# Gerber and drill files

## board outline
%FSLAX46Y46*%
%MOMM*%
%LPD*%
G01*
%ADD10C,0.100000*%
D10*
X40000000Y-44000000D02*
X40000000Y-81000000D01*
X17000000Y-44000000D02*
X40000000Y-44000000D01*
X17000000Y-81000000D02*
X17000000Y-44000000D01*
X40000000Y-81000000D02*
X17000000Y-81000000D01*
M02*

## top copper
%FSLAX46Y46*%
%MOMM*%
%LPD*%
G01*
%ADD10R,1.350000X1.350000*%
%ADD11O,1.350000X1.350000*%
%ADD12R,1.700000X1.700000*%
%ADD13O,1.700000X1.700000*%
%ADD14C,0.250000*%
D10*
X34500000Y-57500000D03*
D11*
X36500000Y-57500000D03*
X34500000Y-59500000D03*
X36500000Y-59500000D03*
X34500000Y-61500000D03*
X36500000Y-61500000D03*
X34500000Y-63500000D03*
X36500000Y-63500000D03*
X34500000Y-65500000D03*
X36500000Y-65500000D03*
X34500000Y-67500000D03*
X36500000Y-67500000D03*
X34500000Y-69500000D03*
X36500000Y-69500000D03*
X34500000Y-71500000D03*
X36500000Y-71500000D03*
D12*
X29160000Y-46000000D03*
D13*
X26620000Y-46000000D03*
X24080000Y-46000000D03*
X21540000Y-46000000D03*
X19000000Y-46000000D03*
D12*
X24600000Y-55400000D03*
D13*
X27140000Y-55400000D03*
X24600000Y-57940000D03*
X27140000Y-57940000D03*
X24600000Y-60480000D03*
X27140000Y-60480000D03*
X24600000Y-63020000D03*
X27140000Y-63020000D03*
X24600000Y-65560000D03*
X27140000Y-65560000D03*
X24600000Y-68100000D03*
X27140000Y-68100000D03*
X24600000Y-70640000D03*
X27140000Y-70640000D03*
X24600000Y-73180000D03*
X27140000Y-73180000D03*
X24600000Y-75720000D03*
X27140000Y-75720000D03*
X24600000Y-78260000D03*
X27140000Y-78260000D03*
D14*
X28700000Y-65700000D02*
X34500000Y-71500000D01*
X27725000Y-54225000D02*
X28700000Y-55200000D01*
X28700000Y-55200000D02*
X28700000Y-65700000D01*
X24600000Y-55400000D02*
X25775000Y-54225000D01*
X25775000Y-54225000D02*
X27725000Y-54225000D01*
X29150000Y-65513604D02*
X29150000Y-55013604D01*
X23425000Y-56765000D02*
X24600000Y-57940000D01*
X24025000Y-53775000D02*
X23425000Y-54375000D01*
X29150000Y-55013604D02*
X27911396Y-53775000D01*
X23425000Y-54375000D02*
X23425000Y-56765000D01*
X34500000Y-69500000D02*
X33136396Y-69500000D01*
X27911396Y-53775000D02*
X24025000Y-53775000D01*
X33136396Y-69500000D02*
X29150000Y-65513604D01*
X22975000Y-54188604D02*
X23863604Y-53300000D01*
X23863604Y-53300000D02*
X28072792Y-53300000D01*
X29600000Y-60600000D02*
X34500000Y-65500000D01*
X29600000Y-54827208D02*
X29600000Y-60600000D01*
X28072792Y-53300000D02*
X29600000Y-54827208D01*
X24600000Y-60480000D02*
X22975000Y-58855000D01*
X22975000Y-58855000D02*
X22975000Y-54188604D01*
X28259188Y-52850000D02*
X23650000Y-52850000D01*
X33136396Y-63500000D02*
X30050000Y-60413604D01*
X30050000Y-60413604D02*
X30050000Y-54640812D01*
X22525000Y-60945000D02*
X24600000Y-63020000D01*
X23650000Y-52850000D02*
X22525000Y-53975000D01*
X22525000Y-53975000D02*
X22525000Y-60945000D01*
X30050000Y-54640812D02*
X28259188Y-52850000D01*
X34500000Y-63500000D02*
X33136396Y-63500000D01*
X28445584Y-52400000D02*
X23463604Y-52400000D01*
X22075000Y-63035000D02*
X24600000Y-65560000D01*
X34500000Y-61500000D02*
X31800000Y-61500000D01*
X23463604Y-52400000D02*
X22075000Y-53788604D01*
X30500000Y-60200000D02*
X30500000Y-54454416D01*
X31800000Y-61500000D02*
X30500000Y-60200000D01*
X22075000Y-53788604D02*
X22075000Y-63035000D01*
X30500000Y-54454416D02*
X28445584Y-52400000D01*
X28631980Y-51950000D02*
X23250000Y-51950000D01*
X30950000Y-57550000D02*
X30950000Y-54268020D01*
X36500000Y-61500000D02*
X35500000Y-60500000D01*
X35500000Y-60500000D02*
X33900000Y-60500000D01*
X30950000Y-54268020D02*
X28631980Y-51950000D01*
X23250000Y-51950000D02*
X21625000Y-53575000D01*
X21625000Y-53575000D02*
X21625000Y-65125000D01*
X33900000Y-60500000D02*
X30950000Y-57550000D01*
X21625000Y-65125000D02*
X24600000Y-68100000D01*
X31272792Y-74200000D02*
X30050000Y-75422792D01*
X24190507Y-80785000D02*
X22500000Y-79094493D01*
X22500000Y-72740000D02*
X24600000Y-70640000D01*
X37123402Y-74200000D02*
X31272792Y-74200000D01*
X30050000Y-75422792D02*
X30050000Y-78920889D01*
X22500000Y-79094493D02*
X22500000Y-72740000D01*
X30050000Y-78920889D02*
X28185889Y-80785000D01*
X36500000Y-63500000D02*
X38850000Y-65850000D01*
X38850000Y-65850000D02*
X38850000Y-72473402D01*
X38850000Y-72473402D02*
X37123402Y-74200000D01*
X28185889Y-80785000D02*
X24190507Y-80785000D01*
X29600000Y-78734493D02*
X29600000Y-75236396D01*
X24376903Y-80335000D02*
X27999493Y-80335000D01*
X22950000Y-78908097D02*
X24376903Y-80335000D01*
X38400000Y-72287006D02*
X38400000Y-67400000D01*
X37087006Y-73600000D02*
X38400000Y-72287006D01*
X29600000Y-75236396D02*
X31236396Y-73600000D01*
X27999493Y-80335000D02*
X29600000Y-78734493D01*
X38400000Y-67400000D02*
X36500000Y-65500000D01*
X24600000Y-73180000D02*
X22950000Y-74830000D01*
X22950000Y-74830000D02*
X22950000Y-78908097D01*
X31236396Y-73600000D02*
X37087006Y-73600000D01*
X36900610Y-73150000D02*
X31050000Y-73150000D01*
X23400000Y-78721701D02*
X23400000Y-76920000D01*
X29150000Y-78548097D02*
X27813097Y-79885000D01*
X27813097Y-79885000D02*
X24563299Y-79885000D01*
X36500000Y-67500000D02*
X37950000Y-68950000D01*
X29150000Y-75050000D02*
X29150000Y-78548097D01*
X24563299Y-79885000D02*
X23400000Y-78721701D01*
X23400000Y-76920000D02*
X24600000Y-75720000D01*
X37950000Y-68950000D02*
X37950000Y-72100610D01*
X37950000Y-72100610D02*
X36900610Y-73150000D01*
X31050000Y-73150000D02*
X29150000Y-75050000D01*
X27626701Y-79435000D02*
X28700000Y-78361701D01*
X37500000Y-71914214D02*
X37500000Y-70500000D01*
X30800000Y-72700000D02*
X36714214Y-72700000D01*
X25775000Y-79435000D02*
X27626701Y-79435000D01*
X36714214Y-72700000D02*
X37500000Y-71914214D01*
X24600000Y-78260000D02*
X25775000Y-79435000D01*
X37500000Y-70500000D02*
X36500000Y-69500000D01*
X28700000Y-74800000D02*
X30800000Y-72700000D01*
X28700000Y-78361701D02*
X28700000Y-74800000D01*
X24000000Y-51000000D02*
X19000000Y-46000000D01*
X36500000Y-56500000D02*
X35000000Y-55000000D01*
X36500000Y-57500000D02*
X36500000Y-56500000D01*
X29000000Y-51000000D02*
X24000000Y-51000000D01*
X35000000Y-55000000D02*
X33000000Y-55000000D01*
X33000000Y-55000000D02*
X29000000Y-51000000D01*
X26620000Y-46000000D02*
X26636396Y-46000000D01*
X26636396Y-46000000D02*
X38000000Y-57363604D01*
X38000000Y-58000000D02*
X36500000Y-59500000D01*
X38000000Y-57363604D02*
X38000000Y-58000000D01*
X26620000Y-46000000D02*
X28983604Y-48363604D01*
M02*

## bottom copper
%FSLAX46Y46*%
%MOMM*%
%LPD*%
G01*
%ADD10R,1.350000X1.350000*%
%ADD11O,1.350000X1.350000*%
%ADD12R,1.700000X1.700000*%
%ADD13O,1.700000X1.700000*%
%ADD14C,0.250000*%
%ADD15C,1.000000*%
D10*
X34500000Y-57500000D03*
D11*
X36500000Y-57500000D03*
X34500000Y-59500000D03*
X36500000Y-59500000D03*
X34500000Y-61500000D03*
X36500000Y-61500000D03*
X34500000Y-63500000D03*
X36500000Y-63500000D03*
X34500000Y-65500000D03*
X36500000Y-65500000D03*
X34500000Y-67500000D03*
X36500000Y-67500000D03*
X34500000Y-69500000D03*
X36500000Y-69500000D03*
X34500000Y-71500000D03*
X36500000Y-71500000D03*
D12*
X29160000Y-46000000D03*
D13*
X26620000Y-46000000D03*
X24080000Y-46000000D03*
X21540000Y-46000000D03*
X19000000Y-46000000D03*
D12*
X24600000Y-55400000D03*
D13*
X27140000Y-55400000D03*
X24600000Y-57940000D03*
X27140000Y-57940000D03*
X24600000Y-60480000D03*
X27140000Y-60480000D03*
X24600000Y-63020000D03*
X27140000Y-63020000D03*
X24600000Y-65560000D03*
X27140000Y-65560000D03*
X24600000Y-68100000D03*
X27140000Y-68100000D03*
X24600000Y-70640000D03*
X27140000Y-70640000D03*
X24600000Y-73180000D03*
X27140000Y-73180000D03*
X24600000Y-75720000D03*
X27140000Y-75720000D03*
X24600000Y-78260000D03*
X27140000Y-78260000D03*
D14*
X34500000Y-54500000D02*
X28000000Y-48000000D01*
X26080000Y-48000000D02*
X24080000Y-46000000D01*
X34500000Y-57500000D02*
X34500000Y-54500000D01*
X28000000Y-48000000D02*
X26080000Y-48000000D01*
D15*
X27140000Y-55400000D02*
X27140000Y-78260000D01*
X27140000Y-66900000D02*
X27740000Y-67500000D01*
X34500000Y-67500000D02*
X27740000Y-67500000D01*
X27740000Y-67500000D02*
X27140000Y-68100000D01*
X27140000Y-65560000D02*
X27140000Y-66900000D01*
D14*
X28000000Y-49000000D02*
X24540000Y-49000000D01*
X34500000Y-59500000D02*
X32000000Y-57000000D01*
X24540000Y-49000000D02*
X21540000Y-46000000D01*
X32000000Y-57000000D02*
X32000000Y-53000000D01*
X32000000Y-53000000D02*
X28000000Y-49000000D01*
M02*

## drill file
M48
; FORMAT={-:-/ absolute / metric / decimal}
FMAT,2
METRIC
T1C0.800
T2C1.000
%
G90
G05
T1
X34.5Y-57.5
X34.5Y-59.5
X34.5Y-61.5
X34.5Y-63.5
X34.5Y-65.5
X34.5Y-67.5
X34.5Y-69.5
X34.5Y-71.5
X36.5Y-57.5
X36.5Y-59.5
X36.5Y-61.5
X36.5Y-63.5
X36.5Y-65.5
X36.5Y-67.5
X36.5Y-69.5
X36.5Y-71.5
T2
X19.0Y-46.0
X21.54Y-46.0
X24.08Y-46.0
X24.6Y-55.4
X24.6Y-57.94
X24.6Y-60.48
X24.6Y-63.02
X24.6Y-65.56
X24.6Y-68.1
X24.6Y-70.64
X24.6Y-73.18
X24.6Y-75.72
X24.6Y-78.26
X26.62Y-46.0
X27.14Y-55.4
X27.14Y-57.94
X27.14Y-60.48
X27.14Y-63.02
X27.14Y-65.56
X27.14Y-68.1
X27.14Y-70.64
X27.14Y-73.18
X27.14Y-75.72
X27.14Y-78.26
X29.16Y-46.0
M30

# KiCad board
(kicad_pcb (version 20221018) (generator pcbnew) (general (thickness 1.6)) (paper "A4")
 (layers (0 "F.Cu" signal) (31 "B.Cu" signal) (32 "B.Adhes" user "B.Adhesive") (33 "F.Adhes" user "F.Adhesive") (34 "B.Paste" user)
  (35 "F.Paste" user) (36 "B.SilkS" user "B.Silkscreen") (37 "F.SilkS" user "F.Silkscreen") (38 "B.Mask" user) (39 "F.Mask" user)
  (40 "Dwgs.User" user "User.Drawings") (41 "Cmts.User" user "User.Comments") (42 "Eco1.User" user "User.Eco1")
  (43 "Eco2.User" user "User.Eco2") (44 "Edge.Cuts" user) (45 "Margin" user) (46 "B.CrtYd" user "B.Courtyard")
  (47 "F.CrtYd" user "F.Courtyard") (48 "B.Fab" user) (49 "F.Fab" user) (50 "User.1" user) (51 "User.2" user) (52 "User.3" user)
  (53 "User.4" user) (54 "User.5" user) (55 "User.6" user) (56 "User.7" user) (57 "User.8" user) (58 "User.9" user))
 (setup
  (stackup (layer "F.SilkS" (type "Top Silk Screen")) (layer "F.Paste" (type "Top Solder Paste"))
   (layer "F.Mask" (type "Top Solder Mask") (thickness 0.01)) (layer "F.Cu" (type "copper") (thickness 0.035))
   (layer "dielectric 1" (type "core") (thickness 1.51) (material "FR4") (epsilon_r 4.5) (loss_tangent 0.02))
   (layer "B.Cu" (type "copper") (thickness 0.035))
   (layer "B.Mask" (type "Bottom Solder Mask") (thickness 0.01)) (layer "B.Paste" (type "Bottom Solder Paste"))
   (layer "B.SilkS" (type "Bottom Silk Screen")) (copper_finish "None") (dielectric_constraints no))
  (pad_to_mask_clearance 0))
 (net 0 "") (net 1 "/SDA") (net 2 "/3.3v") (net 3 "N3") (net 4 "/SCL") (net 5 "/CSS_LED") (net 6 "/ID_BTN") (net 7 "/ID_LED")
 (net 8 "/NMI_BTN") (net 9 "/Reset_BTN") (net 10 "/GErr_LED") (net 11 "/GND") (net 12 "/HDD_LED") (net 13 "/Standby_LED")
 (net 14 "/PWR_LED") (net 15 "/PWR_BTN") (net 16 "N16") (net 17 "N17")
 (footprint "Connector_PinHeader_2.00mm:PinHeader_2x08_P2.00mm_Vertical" (layer "F.Cu") (at 34.5 57.5)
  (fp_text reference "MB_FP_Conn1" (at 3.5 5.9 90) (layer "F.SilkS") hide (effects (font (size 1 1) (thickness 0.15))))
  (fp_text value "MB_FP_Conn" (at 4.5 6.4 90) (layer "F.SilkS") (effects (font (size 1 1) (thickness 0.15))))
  (pad "1" thru_hole rect (at 0 0) (size 1.35 1.35) (drill 0.8) (layers "*.Cu" "*.Mask") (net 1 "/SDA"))
  (pad "2" thru_hole oval (at 2 0) (size 1.35 1.35) (drill 0.8) (layers "*.Cu" "*.Mask") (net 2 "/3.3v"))
  (pad "3" thru_hole oval (at 0 2) (size 1.35 1.35) (drill 0.8) (layers "*.Cu" "*.Mask") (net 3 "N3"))
  (pad "4" thru_hole oval (at 2 2) (size 1.35 1.35) (drill 0.8) (layers "*.Cu" "*.Mask") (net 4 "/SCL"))
  (pad "5" thru_hole oval (at 0 4) (size 1.35 1.35) (drill 0.8) (layers "*.Cu" "*.Mask") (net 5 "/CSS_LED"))
  (pad "6" thru_hole oval (at 2 4) (size 1.35 1.35) (drill 0.8) (layers "*.Cu" "*.Mask") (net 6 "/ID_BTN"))
  (pad "7" thru_hole oval (at 0 6) (size 1.35 1.35) (drill 0.8) (layers "*.Cu" "*.Mask") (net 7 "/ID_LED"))
  (pad "8" thru_hole oval (at 2 6) (size 1.35 1.35) (drill 0.8) (layers "*.Cu" "*.Mask") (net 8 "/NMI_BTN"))
  (pad "9" thru_hole oval (at 0 8) (size 1.35 1.35) (drill 0.8) (layers "*.Cu" "*.Mask") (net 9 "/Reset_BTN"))
  (pad "10" thru_hole oval (at 2 8) (size 1.35 1.35) (drill 0.8) (layers "*.Cu" "*.Mask") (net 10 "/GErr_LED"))
  (pad "11" thru_hole oval (at 0 10) (size 1.35 1.35) (drill 0.8) (layers "*.Cu" "*.Mask") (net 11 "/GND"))
  (pad "12" thru_hole oval (at 2 10) (size 1.35 1.35) (drill 0.8) (layers "*.Cu" "*.Mask") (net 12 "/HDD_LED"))
  (pad "13" thru_hole oval (at 0 12) (size 1.35 1.35) (drill 0.8) (layers "*.Cu" "*.Mask") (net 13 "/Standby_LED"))
  (pad "14" thru_hole oval (at 2 12) (size 1.35 1.35) (drill 0.8) (layers "*.Cu" "*.Mask") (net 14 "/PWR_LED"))
  (pad "15" thru_hole oval (at 0 14) (size 1.35 1.35) (drill 0.8) (layers "*.Cu" "*.Mask") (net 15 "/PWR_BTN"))
  (pad "16" thru_hole oval (at 2 14) (size 1.35 1.35) (drill 0.8) (layers "*.Cu" "*.Mask") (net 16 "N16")))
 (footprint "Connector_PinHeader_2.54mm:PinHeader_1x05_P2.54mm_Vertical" (layer "F.Cu") (at 29.16 46 -90)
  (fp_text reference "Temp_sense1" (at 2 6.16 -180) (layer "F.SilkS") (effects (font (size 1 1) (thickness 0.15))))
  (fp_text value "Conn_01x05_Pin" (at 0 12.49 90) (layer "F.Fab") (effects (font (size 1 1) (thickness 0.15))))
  (pad "1" thru_hole rect (at 0 0 270) (size 1.7 1.7) (drill 1) (layers "*.Cu" "*.Mask") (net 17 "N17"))
  (pad "2" thru_hole oval (at 0 2.54 270) (size 1.7 1.7) (drill 1) (layers "*.Cu" "*.Mask") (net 4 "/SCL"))
  (pad "3" thru_hole oval (at 0 5.08 270) (size 1.7 1.7) (drill 1) (layers "*.Cu" "*.Mask") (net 1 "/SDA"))
  (pad "4" thru_hole oval (at 0 7.62 270) (size 1.7 1.7) (drill 1) (layers "*.Cu" "*.Mask") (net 3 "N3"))
  (pad "5" thru_hole oval (at 0 10.16 270) (size 1.7 1.7) (drill 1) (layers "*.Cu" "*.Mask") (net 2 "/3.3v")))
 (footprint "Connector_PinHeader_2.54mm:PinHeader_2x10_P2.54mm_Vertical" (layer "F.Cu") (at 24.6 55.4)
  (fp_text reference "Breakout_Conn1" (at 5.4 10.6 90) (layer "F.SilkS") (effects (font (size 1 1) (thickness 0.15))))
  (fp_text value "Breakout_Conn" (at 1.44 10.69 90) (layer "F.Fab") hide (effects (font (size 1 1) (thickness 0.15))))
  (pad "1" thru_hole rect (at 0 0) (size 1.7 1.7) (drill 1) (layers "*.Cu" "*.Mask") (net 15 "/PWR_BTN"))
  (pad "2" thru_hole oval (at 2.54 0) (size 1.7 1.7) (drill 1) (layers "*.Cu" "*.Mask") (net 11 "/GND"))
  (pad "3" thru_hole oval (at 0 2.54) (size 1.7 1.7) (drill 1) (layers "*.Cu" "*.Mask") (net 13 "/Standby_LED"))
  (pad "4" thru_hole oval (at 2.54 2.54) (size 1.7 1.7) (drill 1) (layers "*.Cu" "*.Mask") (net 11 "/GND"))
  (pad "5" thru_hole oval (at 0 5.08) (size 1.7 1.7) (drill 1) (layers "*.Cu" "*.Mask") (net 9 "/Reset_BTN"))
  (pad "6" thru_hole oval (at 2.54 5.08) (size 1.7 1.7) (drill 1) (layers "*.Cu" "*.Mask") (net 11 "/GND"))
  (pad "7" thru_hole oval (at 0 7.62) (size 1.7 1.7) (drill 1) (layers "*.Cu" "*.Mask") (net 7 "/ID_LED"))
  (pad "8" thru_hole oval (at 2.54 7.62) (size 1.7 1.7) (drill 1) (layers "*.Cu" "*.Mask") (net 11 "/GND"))
  (pad "9" thru_hole oval (at 0 10.16) (size 1.7 1.7) (drill 1) (layers "*.Cu" "*.Mask") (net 5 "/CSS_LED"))
  (pad "10" thru_hole oval (at 2.54 10.16) (size 1.7 1.7) (drill 1) (layers "*.Cu" "*.Mask") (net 11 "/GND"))
  (pad "11" thru_hole oval (at 0 12.7) (size 1.7 1.7) (drill 1) (layers "*.Cu" "*.Mask") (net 6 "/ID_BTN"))
  (pad "12" thru_hole oval (at 2.54 12.7) (size 1.7 1.7) (drill 1) (layers "*.Cu" "*.Mask") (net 11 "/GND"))
  (pad "13" thru_hole oval (at 0 15.24) (size 1.7 1.7) (drill 1) (layers "*.Cu" "*.Mask") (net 8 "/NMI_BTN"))
  (pad "14" thru_hole oval (at 2.54 15.24) (size 1.7 1.7) (drill 1) (layers "*.Cu" "*.Mask") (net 11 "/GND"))
  (pad "15" thru_hole oval (at 0 17.78) (size 1.7 1.7) (drill 1) (layers "*.Cu" "*.Mask") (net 10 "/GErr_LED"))
  (pad "16" thru_hole oval (at 2.54 17.78) (size 1.7 1.7) (drill 1) (layers "*.Cu" "*.Mask") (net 11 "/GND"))
  (pad "17" thru_hole oval (at 0 20.32) (size 1.7 1.7) (drill 1) (layers "*.Cu" "*.Mask") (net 12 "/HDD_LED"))
  (pad "18" thru_hole oval (at 2.54 20.32) (size 1.7 1.7) (drill 1) (layers "*.Cu" "*.Mask") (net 11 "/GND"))
  (pad "19" thru_hole oval (at 0 22.86) (size 1.7 1.7) (drill 1) (layers "*.Cu" "*.Mask") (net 14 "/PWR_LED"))
  (pad "20" thru_hole oval (at 2.54 22.86) (size 1.7 1.7) (drill 1) (layers "*.Cu" "*.Mask") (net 11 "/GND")))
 (gr_line (start 40 44) (end 40 81) (stroke (width 0.1) (type default)) (layer "Edge.Cuts"))
 (gr_line (start 17 44) (end 40 44) (stroke (width 0.1) (type default)) (layer "Edge.Cuts"))
 (gr_line (start 17 81) (end 17 44) (stroke (width 0.1) (type default)) (layer "Edge.Cuts"))
 (gr_line (start 40 81) (end 17 81) (stroke (width 0.1) (type default)) (layer "Edge.Cuts"))
 (segment (start 34.5 54.5) (end 28 48) (width 0.25) (layer "B.Cu") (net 1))
 (segment (start 26.08 48) (end 24.08 46) (width 0.25) (layer "B.Cu") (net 1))
 (segment (start 34.5 57.5) (end 34.5 54.5) (width 0.25) (layer "B.Cu") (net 1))
 (segment (start 28 48) (end 26.08 48) (width 0.25) (layer "B.Cu") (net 1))
 (segment (start 28.7 65.7) (end 34.5 71.5) (width 0.25) (layer "F.Cu") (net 15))
 (segment (start 27.725 54.225) (end 28.7 55.2) (width 0.25) (layer "F.Cu") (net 15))
 (segment (start 28.7 55.2) (end 28.7 65.7) (width 0.25) (layer "F.Cu") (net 15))
 (segment (start 24.6 55.4) (end 25.775 54.225) (width 0.25) (layer "F.Cu") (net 15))
 (segment (start 25.775 54.225) (end 27.725 54.225) (width 0.25) (layer "F.Cu") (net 15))
 (segment (start 27.14 55.4) (end 27.14 78.26) (width 1) (layer "B.Cu") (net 11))
 (segment (start 27.14 66.9) (end 27.74 67.5) (width 1) (layer "B.Cu") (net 11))
 (segment (start 34.5 67.5) (end 27.74 67.5) (width 1) (layer "B.Cu") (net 11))
 (segment (start 27.74 67.5) (end 27.14 68.1) (width 1) (layer "B.Cu") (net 11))
 (segment (start 27.14 65.56) (end 27.14 66.9) (width 1) (layer "B.Cu") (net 11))
 (segment (start 29.15 65.513604) (end 29.15 55.013604) (width 0.25) (layer "F.Cu") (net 13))
 (segment (start 23.425 56.765) (end 24.6 57.94) (width 0.25) (layer "F.Cu") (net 13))
 (segment (start 24.025 53.775) (end 23.425 54.375) (width 0.25) (layer "F.Cu") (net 13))
 (segment (start 29.15 55.013604) (end 27.911396 53.775) (width 0.25) (layer "F.Cu") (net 13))
 (segment (start 23.425 54.375) (end 23.425 56.765) (width 0.25) (layer "F.Cu") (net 13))
 (segment (start 34.5 69.5) (end 33.136396 69.5) (width 0.25) (layer "F.Cu") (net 13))
 (segment (start 27.911396 53.775) (end 24.025 53.775) (width 0.25) (layer "F.Cu") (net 13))
 (segment (start 33.136396 69.5) (end 29.15 65.513604) (width 0.25) (layer "F.Cu") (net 13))
 (segment (start 22.975 54.188604) (end 23.863604 53.3) (width 0.25) (layer "F.Cu") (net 9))
 (segment (start 23.863604 53.3) (end 28.072792 53.3) (width 0.25) (layer "F.Cu") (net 9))
 (segment (start 29.6 60.6) (end 34.5 65.5) (width 0.25) (layer "F.Cu") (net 9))
 (segment (start 29.6 54.827208) (end 29.6 60.6) (width 0.25) (layer "F.Cu") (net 9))
 (segment (start 28.072792 53.3) (end 29.6 54.827208) (width 0.25) (layer "F.Cu") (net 9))
 (segment (start 24.6 60.48) (end 22.975 58.855) (width 0.25) (layer "F.Cu") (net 9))
 (segment (start 22.975 58.855) (end 22.975 54.188604) (width 0.25) (layer "F.Cu") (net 9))
 (segment (start 28.259188 52.85) (end 23.65 52.85) (width 0.25) (layer "F.Cu") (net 7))
 (segment (start 33.136396 63.5) (end 30.05 60.413604) (width 0.25) (layer "F.Cu") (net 7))
 (segment (start 30.05 60.413604) (end 30.05 54.640812) (width 0.25) (layer "F.Cu") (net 7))
 (segment (start 22.525 60.945) (end 24.6 63.02) (width 0.25) (layer "F.Cu") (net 7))
 (segment (start 23.65 52.85) (end 22.525 53.975) (width 0.25) (layer "F.Cu") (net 7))
 (segment (start 22.525 53.975) (end 22.525 60.945) (width 0.25) (layer "F.Cu") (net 7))
 (segment (start 30.05 54.640812) (end 28.259188 52.85) (width 0.25) (layer "F.Cu") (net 7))
 (segment (start 34.5 63.5) (end 33.136396 63.5) (width 0.25) (layer "F.Cu") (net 7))
 (segment (start 28.445584 52.4) (end 23.463604 52.4) (width 0.25) (layer "F.Cu") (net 5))
 (segment (start 22.075 63.035) (end 24.6 65.56) (width 0.25) (layer "F.Cu") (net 5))
 (segment (start 34.5 61.5) (end 31.8 61.5) (width 0.25) (layer "F.Cu") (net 5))
 (segment (start 23.463604 52.4) (end 22.075 53.788604) (width 0.25) (layer "F.Cu") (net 5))
 (segment (start 30.5 60.2) (end 30.5 54.454416) (width 0.25) (layer "F.Cu") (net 5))
 (segment (start 31.8 61.5) (end 30.5 60.2) (width 0.25) (layer "F.Cu") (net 5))
 (segment (start 22.075 53.788604) (end 22.075 63.035) (width 0.25) (layer "F.Cu") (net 5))
 (segment (start 30.5 54.454416) (end 28.445584 52.4) (width 0.25) (layer "F.Cu") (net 5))
 (segment (start 28.63198 51.95) (end 23.25 51.95) (width 0.25) (layer "F.Cu") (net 6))
 (segment (start 30.95 57.55) (end 30.95 54.26802) (width 0.25) (layer "F.Cu") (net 6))
 (segment (start 36.5 61.5) (end 35.5 60.5) (width 0.25) (layer "F.Cu") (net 6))
 (segment (start 35.5 60.5) (end 33.9 60.5) (width 0.25) (layer "F.Cu") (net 6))
 (segment (start 30.95 54.26802) (end 28.63198 51.95) (width 0.25) (layer "F.Cu") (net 6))
 (segment (start 23.25 51.95) (end 21.625 53.575) (width 0.25) (layer "F.Cu") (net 6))
 (segment (start 21.625 53.575) (end 21.625 65.125) (width 0.25) (layer "F.Cu") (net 6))
 (segment (start 33.9 60.5) (end 30.95 57.55) (width 0.25) (layer "F.Cu") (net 6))
 (segment (start 21.625 65.125) (end 24.6 68.1) (width 0.25) (layer "F.Cu") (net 6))
 (segment (start 31.272792 74.2) (end 30.05 75.422792) (width 0.25) (layer "F.Cu") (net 8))
 (segment (start 24.190507 80.785) (end 22.5 79.094493) (width 0.25) (layer "F.Cu") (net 8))
 (segment (start 22.5 72.74) (end 24.6 70.64) (width 0.25) (layer "F.Cu") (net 8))
 (segment (start 37.123402 74.2) (end 31.272792 74.2) (width 0.25) (layer "F.Cu") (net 8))
 (segment (start 30.05 75.422792) (end 30.05 78.920889) (width 0.25) (layer "F.Cu") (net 8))
 (segment (start 22.5 79.094493) (end 22.5 72.74) (width 0.25) (layer "F.Cu") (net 8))
 (segment (start 30.05 78.920889) (end 28.185889 80.785) (width 0.25) (layer "F.Cu") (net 8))
 (segment (start 36.5 63.5) (end 38.85 65.85) (width 0.25) (layer "F.Cu") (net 8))
 (segment (start 38.85 65.85) (end 38.85 72.473402) (width 0.25) (layer "F.Cu") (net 8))
 (segment (start 38.85 72.473402) (end 37.123402 74.2) (width 0.25) (layer "F.Cu") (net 8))
 (segment (start 28.185889 80.785) (end 24.190507 80.785) (width 0.25) (layer "F.Cu") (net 8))
 (segment (start 29.6 78.734493) (end 29.6 75.236396) (width 0.25) (layer "F.Cu") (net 10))
 (segment (start 24.376903 80.335) (end 27.999493 80.335) (width 0.25) (layer "F.Cu") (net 10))
 (segment (start 22.95 78.908097) (end 24.376903 80.335) (width 0.25) (layer "F.Cu") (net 10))
 (segment (start 38.4 72.287006) (end 38.4 67.4) (width 0.25) (layer "F.Cu") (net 10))
 (segment (start 37.087006 73.6) (end 38.4 72.287006) (width 0.25) (layer "F.Cu") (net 10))
 (segment (start 29.6 75.236396) (end 31.236396 73.6) (width 0.25) (layer "F.Cu") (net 10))
 (segment (start 27.999493 80.335) (end 29.6 78.734493) (width 0.25) (layer "F.Cu") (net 10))
 (segment (start 38.4 67.4) (end 36.5 65.5) (width 0.25) (layer "F.Cu") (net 10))
 (segment (start 24.6 73.18) (end 22.95 74.83) (width 0.25) (layer "F.Cu") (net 10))
 (segment (start 22.95 74.83) (end 22.95 78.908097) (width 0.25) (layer "F.Cu") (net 10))
 (segment (start 31.236396 73.6) (end 37.087006 73.6) (width 0.25) (layer "F.Cu") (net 10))
 (segment (start 36.90061 73.15) (end 31.05 73.15) (width 0.25) (layer "F.Cu") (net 12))
 (segment (start 23.4 78.721701) (end 23.4 76.92) (width 0.25) (layer "F.Cu") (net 12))
 (segment (start 29.15 78.548097) (end 27.813097 79.885) (width 0.25) (layer "F.Cu") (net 12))
 (segment (start 27.813097 79.885) (end 24.563299 79.885) (width 0.25) (layer "F.Cu") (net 12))
 (segment (start 36.5 67.5) (end 37.95 68.95) (width 0.25) (layer "F.Cu") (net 12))
 (segment (start 29.15 75.05) (end 29.15 78.548097) (width 0.25) (layer "F.Cu") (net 12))
 (segment (start 24.563299 79.885) (end 23.4 78.721701) (width 0.25) (layer "F.Cu") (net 12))
 (segment (start 23.4 76.92) (end 24.6 75.72) (width 0.25) (layer "F.Cu") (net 12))
 (segment (start 37.95 68.95) (end 37.95 72.10061) (width 0.25) (layer "F.Cu") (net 12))
 (segment (start 37.95 72.10061) (end 36.90061 73.15) (width 0.25) (layer "F.Cu") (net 12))
 (segment (start 31.05 73.15) (end 29.15 75.05) (width 0.25) (layer "F.Cu") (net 12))
 (segment (start 27.626701 79.435) (end 28.7 78.361701) (width 0.25) (layer "F.Cu") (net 14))
 (segment (start 37.5 71.914214) (end 37.5 70.5) (width 0.25) (layer "F.Cu") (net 14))
 (segment (start 30.8 72.7) (end 36.714214 72.7) (width 0.25) (layer "F.Cu") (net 14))
 (segment (start 25.775 79.435) (end 27.626701 79.435) (width 0.25) (layer "F.Cu") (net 14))
 (segment (start 36.714214 72.7) (end 37.5 71.914214) (width 0.25) (layer "F.Cu") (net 14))
 (segment (start 24.6 78.26) (end 25.775 79.435) (width 0.25) (layer "F.Cu") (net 14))
 (segment (start 37.5 70.5) (end 36.5 69.5) (width 0.25) (layer "F.Cu") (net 14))
 (segment (start 28.7 74.8) (end 30.8 72.7) (width 0.25) (layer "F.Cu") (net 14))
 (segment (start 28.7 78.361701) (end 28.7 74.8) (width 0.25) (layer "F.Cu") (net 14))
 (segment (start 24 51) (end 19 46) (width 0.25) (layer "F.Cu") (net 2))
 (segment (start 36.5 56.5) (end 35 55) (width 0.25) (layer "F.Cu") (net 2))
 (segment (start 36.5 57.5) (end 36.5 56.5) (width 0.25) (layer "F.Cu") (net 2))
 (segment (start 29 51) (end 24 51) (width 0.25) (layer "F.Cu") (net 2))
 (segment (start 35 55) (end 33 55) (width 0.25) (layer "F.Cu") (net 2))
 (segment (start 33 55) (end 29 51) (width 0.25) (layer "F.Cu") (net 2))
 (segment (start 26.62 46) (end 26.636396 46) (width 0.25) (layer "F.Cu") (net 4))
 (segment (start 26.636396 46) (end 38 57.363604) (width 0.25) (layer "F.Cu") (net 4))
 (segment (start 38 58) (end 36.5 59.5) (width 0.25) (layer "F.Cu") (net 4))
 (segment (start 38 57.363604) (end 38 58) (width 0.25) (layer "F.Cu") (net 4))
 (segment (start 26.62 46) (end 28.983604 48.363604) (width 0.25) (layer "F.Cu") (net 4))
 (segment (start 28 49) (end 24.54 49) (width 0.25) (layer "B.Cu") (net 3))
 (segment (start 34.5 59.5) (end 32 57) (width 0.25) (layer "B.Cu") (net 3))
 (segment (start 24.54 49) (end 21.54 46) (width 0.25) (layer "B.Cu") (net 3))
 (segment (start 32 57) (end 32 53) (width 0.25) (layer "B.Cu") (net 3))
 (segment (start 32 53) (end 28 49) (width 0.25) (layer "B.Cu") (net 3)))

